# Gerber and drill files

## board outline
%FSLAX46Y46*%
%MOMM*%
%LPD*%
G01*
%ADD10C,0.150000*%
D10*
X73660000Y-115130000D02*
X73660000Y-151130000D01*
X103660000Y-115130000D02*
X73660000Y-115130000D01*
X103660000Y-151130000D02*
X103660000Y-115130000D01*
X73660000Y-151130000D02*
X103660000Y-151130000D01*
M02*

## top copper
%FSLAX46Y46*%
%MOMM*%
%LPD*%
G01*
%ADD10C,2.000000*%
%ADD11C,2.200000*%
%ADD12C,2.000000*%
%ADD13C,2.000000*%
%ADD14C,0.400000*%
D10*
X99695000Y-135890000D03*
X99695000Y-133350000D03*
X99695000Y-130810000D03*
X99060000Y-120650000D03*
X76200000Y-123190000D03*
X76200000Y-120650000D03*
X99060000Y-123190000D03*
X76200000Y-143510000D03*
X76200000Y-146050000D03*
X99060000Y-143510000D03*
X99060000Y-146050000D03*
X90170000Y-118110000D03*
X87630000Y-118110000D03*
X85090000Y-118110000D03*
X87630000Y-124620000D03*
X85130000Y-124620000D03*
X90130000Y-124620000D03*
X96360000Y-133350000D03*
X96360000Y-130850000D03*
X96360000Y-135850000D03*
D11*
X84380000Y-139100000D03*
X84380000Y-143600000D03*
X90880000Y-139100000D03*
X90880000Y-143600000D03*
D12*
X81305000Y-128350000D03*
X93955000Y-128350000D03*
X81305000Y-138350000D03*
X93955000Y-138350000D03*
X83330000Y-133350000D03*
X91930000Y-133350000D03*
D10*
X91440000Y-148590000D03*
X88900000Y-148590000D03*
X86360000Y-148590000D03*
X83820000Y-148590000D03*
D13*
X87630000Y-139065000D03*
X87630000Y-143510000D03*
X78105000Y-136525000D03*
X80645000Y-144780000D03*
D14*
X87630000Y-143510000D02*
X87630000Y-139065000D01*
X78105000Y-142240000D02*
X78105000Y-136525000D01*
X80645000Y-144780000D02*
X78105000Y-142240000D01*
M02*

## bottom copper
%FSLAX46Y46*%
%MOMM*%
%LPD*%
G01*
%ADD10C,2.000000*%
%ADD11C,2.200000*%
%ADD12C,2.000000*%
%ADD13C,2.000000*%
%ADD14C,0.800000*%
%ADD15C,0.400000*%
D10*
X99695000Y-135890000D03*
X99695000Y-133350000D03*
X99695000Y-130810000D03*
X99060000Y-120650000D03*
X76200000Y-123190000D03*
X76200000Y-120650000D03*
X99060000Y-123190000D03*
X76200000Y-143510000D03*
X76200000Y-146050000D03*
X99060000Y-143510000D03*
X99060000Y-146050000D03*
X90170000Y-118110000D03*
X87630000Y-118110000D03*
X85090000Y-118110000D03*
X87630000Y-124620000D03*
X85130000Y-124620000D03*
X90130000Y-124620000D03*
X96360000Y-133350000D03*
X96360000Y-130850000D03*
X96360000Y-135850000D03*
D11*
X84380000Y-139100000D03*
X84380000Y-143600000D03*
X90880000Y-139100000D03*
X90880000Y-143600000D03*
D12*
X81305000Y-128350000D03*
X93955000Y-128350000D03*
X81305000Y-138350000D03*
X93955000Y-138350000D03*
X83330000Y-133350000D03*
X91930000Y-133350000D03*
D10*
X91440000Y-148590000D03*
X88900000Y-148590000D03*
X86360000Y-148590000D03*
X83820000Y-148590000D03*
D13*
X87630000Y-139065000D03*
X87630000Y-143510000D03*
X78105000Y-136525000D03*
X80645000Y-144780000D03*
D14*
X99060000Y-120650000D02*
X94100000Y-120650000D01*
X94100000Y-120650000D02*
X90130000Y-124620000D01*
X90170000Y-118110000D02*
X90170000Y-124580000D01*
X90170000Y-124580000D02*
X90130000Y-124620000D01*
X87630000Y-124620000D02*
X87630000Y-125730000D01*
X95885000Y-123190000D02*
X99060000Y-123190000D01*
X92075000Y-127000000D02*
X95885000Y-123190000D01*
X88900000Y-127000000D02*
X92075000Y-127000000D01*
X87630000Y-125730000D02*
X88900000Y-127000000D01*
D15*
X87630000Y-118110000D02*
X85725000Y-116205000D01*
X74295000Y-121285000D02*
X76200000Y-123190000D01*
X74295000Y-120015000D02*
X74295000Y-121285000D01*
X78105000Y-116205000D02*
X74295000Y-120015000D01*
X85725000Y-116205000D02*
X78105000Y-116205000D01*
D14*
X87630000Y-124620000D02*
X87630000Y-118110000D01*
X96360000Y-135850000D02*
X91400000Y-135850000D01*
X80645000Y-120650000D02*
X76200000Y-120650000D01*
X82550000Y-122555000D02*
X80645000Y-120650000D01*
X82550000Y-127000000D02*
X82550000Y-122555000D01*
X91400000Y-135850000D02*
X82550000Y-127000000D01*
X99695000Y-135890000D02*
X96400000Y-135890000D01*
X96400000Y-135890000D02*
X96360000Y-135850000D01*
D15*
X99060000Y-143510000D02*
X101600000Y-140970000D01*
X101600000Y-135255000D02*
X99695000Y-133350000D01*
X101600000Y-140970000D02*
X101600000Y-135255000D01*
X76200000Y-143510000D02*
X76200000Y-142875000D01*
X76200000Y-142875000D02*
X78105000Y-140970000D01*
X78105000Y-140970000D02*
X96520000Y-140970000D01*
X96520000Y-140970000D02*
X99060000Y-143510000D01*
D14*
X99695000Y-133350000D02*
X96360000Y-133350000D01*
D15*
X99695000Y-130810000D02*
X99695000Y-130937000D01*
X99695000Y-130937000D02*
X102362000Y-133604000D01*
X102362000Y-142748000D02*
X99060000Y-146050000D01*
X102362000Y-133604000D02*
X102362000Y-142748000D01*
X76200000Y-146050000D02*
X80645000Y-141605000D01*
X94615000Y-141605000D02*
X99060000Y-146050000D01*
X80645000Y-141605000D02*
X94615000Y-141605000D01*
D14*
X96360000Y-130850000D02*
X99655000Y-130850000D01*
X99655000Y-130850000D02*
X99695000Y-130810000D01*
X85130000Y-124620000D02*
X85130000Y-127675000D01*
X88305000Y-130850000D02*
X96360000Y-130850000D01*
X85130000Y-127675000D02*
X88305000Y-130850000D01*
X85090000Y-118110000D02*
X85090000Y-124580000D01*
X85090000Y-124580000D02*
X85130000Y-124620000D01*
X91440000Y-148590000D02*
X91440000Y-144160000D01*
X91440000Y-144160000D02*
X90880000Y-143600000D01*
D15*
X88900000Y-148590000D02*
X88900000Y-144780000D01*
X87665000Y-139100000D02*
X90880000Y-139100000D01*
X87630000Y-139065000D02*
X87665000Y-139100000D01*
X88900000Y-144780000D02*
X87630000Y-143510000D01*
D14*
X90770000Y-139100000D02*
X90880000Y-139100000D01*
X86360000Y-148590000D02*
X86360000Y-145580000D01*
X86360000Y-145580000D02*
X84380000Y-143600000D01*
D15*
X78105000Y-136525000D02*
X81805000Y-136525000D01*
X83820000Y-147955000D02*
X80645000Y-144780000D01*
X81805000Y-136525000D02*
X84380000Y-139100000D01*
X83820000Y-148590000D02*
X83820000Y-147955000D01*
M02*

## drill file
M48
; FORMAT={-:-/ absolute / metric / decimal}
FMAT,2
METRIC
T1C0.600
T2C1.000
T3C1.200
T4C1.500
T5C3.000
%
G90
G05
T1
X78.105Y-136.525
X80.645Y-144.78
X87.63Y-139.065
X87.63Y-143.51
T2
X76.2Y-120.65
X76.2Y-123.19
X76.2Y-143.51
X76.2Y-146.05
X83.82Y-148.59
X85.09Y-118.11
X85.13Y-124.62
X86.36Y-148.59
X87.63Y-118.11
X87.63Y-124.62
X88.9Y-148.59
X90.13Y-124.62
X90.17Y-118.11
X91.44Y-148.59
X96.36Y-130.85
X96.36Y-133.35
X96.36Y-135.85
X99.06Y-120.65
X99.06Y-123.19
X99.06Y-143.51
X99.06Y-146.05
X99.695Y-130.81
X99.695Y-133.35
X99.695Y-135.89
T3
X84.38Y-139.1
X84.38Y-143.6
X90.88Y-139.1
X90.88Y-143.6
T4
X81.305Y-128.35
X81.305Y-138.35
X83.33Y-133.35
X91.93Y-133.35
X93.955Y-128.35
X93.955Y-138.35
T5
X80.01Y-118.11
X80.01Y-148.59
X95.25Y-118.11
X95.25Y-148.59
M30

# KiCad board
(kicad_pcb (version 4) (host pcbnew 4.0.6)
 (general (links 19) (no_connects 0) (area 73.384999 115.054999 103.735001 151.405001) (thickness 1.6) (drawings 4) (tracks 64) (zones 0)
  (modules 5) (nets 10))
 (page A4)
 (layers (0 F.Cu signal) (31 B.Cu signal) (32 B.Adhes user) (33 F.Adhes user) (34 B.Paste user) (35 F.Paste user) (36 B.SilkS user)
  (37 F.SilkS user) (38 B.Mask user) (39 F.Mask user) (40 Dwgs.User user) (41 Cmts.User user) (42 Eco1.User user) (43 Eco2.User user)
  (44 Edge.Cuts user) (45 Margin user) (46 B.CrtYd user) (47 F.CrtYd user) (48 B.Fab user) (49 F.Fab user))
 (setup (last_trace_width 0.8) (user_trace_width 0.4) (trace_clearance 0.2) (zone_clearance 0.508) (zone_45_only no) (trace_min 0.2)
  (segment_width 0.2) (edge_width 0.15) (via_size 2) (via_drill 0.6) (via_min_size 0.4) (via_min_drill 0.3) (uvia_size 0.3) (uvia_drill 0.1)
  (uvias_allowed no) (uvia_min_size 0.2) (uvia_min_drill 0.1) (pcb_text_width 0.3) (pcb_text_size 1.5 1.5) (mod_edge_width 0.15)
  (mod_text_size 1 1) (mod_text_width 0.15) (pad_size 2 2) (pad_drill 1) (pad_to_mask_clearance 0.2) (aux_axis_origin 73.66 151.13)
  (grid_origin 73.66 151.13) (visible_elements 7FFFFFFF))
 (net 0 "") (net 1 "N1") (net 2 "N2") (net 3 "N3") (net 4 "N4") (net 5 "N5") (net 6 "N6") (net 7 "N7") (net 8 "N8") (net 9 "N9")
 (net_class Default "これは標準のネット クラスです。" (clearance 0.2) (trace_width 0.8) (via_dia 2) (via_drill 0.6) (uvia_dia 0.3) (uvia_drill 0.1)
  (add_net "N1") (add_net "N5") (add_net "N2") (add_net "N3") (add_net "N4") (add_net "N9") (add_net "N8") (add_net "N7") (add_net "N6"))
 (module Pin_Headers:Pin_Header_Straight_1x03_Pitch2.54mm (layer F.Cu) (at 99.695 135.89 180)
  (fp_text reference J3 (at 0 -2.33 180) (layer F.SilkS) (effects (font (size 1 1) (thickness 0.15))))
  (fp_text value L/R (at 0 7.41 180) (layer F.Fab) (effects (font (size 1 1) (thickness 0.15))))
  (pad 1 thru_hole circle (at 0 0 180) (size 2 2) (drill 1) (layers *.Cu *.Mask) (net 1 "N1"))
  (pad 2 thru_hole circle (at 0 2.54 180) (size 2 2) (drill 1) (layers *.Cu *.Mask) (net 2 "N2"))
  (pad 3 thru_hole circle (at 0 5.08 180) (size 2 2) (drill 1) (layers *.Cu *.Mask) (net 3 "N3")))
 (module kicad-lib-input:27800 (layer F.Cu) (at 87.63 133.35)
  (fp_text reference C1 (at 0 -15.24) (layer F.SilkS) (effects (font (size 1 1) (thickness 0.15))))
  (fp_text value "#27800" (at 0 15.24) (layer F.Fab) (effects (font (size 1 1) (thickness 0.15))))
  (pad 5 thru_hole circle (at 11.43 -12.7) (size 2 2) (drill 1) (layers *.Cu *.Mask) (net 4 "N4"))
  (pad 2 thru_hole circle (at -11.43 -10.16) (size 2 2) (drill 1) (layers *.Cu *.Mask) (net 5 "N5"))
  (pad 1 thru_hole circle (at -11.43 -12.7) (size 2 2) (drill 1) (layers *.Cu *.Mask) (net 1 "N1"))
  (pad 6 thru_hole circle (at 11.43 -10.16) (size 2 2) (drill 1) (layers *.Cu *.Mask) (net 5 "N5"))
  (pad 3 thru_hole circle (at -11.43 10.16) (size 2 2) (drill 1) (layers *.Cu *.Mask) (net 2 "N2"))
  (pad 4 thru_hole circle (at -11.43 12.7) (size 2 2) (drill 1) (layers *.Cu *.Mask) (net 3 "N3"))
  (pad 7 thru_hole circle (at 11.43 10.16) (size 2 2) (drill 1) (layers *.Cu *.Mask) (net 2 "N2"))
  (pad 8 thru_hole circle (at 11.43 12.7) (size 2 2) (drill 1) (layers *.Cu *.Mask) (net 3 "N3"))
  (pad "" np_thru_hole circle (at 7.62 -15.24) (size 3 3) (drill 3) (layers *.Cu *.Mask))
  (pad "" np_thru_hole circle (at -7.62 -15.24) (size 3 3) (drill 3) (layers *.Cu *.Mask))
  (pad "" np_thru_hole circle (at -7.62 15.24) (size 3 3) (drill 3) (layers *.Cu *.Mask))
  (pad "" np_thru_hole circle (at 7.62 15.24) (size 3 3) (drill 3) (layers *.Cu *.Mask)))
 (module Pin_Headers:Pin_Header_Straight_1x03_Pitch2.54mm (layer F.Cu) (at 90.17 118.11 270)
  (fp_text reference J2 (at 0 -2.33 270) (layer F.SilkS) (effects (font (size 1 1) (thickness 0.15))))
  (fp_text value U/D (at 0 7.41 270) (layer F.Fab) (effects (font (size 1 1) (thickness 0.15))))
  (pad 1 thru_hole circle (at 0 0 270) (size 2 2) (drill 1) (layers *.Cu *.Mask) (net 4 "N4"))
  (pad 2 thru_hole circle (at 0 2.54 270) (size 2 2) (drill 1) (layers *.Cu *.Mask) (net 5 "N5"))
  (pad 3 thru_hole circle (at 0 5.08 270) (size 2 2) (drill 1) (layers *.Cu *.Mask) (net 3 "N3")))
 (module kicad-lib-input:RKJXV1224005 (layer F.Cu) (at 87.63 133.35)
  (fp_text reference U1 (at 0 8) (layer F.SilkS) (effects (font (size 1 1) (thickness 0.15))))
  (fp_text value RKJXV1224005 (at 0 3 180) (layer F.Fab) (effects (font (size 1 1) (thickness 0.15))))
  (pad 5 thru_hole circle (at 0 -8.73) (size 2 2) (drill 1) (layers *.Cu *.Mask) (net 5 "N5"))
  (pad 6 thru_hole circle (at -2.5 -8.73) (size 2 2) (drill 1) (layers *.Cu *.Mask) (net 3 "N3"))
  (pad 4 thru_hole circle (at 2.5 -8.73) (size 2 2) (drill 1) (layers *.Cu *.Mask) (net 4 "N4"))
  (pad 2 thru_hole circle (at 8.73 0) (size 2 2) (drill 1) (layers *.Cu *.Mask) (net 2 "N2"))
  (pad 3 thru_hole circle (at 8.73 -2.5) (size 2 2) (drill 1) (layers *.Cu *.Mask) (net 3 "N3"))
  (pad 1 thru_hole circle (at 8.73 2.5) (size 2 2) (drill 1) (layers *.Cu *.Mask) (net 1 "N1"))
  (pad 7 thru_hole circle (at -3.25 5.75) (size 2.2 2.2) (drill 1.2) (layers *.Cu *.Mask) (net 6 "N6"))
  (pad 8 thru_hole circle (at -3.25 10.25) (size 2.2 2.2) (drill 1.2) (layers *.Cu *.Mask) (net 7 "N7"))
  (pad 9 thru_hole circle (at 3.25 5.75) (size 2.2 2.2) (drill 1.2) (layers *.Cu *.Mask) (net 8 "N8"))
  (pad 10 thru_hole circle (at 3.25 10.25) (size 2.2 2.2) (drill 1.2) (layers *.Cu *.Mask) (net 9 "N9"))
  (pad "" np_thru_hole circle (at -6.325 -5) (size 2 2) (drill 1.5) (layers *.Cu *.Mask))
  (pad "" np_thru_hole circle (at 6.325 -5) (size 2 2) (drill 1.5) (layers *.Cu *.Mask))
  (pad "" np_thru_hole circle (at -6.325 5) (size 2 2) (drill 1.5) (layers *.Cu *.Mask))
  (pad "" np_thru_hole circle (at 6.325 5) (size 2 2) (drill 1.5) (layers *.Cu *.Mask))
  (pad "" np_thru_hole circle (at -4.3 0) (size 2 2) (drill 1.5) (layers *.Cu *.Mask))
  (pad "" np_thru_hole circle (at 4.3 0) (size 2 2) (drill 1.5) (layers *.Cu *.Mask)))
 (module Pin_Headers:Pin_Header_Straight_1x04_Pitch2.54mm (layer F.Cu) (at 91.44 148.59 270)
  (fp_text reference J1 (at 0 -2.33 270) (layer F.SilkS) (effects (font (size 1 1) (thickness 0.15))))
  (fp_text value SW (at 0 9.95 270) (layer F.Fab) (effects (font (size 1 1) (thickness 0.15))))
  (pad 1 thru_hole circle (at 0 0 270) (size 2 2) (drill 1) (layers *.Cu *.Mask) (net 9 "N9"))
  (pad 2 thru_hole circle (at 0 2.54 270) (size 2 2) (drill 1) (layers *.Cu *.Mask) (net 8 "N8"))
  (pad 3 thru_hole circle (at 0 5.08 270) (size 2 2) (drill 1) (layers *.Cu *.Mask) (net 7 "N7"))
  (pad 4 thru_hole circle (at 0 7.62 270) (size 2 2) (drill 1) (layers *.Cu *.Mask) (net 6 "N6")))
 (gr_line (start 73.66 115.13) (end 73.66 151.13) (angle 90) (layer Edge.Cuts) (width 0.15))
 (gr_line (start 103.66 115.13) (end 73.66 115.13) (angle 90) (layer Edge.Cuts) (width 0.15))
 (gr_line (start 103.66 151.13) (end 103.66 115.13) (angle 90) (layer Edge.Cuts) (width 0.15))
 (gr_line (start 73.66 151.13) (end 103.66 151.13) (angle 90) (layer Edge.Cuts) (width 0.15))
 (segment (start 99.06 120.65) (end 94.1 120.65) (width 0.8) (layer B.Cu) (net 4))
 (segment (start 94.1 120.65) (end 90.13 124.62) (width 0.8) (layer B.Cu) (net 4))
 (segment (start 90.17 118.11) (end 90.17 124.58) (width 0.8) (layer B.Cu) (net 4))
 (segment (start 90.17 124.58) (end 90.13 124.62) (width 0.8) (layer B.Cu) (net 4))
 (segment (start 87.63 124.62) (end 87.63 125.73) (width 0.8) (layer B.Cu) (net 5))
 (segment (start 95.885 123.19) (end 99.06 123.19) (width 0.8) (layer B.Cu) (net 5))
 (segment (start 92.075 127) (end 95.885 123.19) (width 0.8) (layer B.Cu) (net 5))
 (segment (start 88.9 127) (end 92.075 127) (width 0.8) (layer B.Cu) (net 5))
 (segment (start 87.63 125.73) (end 88.9 127) (width 0.8) (layer B.Cu) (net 5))
 (segment (start 87.63 118.11) (end 85.725 116.205) (width 0.4) (layer B.Cu) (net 5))
 (segment (start 74.295 121.285) (end 76.2 123.19) (width 0.4) (layer B.Cu) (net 5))
 (segment (start 74.295 120.015) (end 74.295 121.285) (width 0.4) (layer B.Cu) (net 5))
 (segment (start 78.105 116.205) (end 74.295 120.015) (width 0.4) (layer B.Cu) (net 5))
 (segment (start 85.725 116.205) (end 78.105 116.205) (width 0.4) (layer B.Cu) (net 5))
 (segment (start 87.63 124.62) (end 87.63 118.11) (width 0.8) (layer B.Cu) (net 5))
 (segment (start 96.36 135.85) (end 91.4 135.85) (width 0.8) (layer B.Cu) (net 1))
 (segment (start 80.645 120.65) (end 76.2 120.65) (width 0.8) (layer B.Cu) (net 1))
 (segment (start 82.55 122.555) (end 80.645 120.65) (width 0.8) (layer B.Cu) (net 1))
 (segment (start 82.55 127) (end 82.55 122.555) (width 0.8) (layer B.Cu) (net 1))
 (segment (start 91.4 135.85) (end 82.55 127) (width 0.8) (layer B.Cu) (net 1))
 (segment (start 99.695 135.89) (end 96.4 135.89) (width 0.8) (layer B.Cu) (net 1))
 (segment (start 96.4 135.89) (end 96.36 135.85) (width 0.8) (layer B.Cu) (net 1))
 (segment (start 99.06 143.51) (end 101.6 140.97) (width 0.4) (layer B.Cu) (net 2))
 (segment (start 101.6 135.255) (end 99.695 133.35) (width 0.4) (layer B.Cu) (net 2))
 (segment (start 101.6 140.97) (end 101.6 135.255) (width 0.4) (layer B.Cu) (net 2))
 (segment (start 76.2 143.51) (end 76.2 142.875) (width 0.4) (layer B.Cu) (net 2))
 (segment (start 76.2 142.875) (end 78.105 140.97) (width 0.4) (layer B.Cu) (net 2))
 (segment (start 78.105 140.97) (end 96.52 140.97) (width 0.4) (layer B.Cu) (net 2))
 (segment (start 96.52 140.97) (end 99.06 143.51) (width 0.4) (layer B.Cu) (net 2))
 (segment (start 99.695 133.35) (end 96.36 133.35) (width 0.8) (layer B.Cu) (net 2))
 (segment (start 99.695 130.81) (end 99.695 130.937) (width 0.4) (layer B.Cu) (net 3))
 (segment (start 99.695 130.937) (end 102.362 133.604) (width 0.4) (layer B.Cu) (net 3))
 (segment (start 102.362 142.748) (end 99.06 146.05) (width 0.4) (layer B.Cu) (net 3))
 (segment (start 102.362 133.604) (end 102.362 142.748) (width 0.4) (layer B.Cu) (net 3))
 (segment (start 76.2 146.05) (end 80.645 141.605) (width 0.4) (layer B.Cu) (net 3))
 (segment (start 94.615 141.605) (end 99.06 146.05) (width 0.4) (layer B.Cu) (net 3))
 (segment (start 80.645 141.605) (end 94.615 141.605) (width 0.4) (layer B.Cu) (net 3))
 (segment (start 96.36 130.85) (end 99.655 130.85) (width 0.8) (layer B.Cu) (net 3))
 (segment (start 99.655 130.85) (end 99.695 130.81) (width 0.8) (layer B.Cu) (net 3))
 (segment (start 85.13 124.62) (end 85.13 127.675) (width 0.8) (layer B.Cu) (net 3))
 (segment (start 88.305 130.85) (end 96.36 130.85) (width 0.8) (layer B.Cu) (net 3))
 (segment (start 85.13 127.675) (end 88.305 130.85) (width 0.8) (layer B.Cu) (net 3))
 (segment (start 85.09 118.11) (end 85.09 124.58) (width 0.8) (layer B.Cu) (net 3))
 (segment (start 85.09 124.58) (end 85.13 124.62) (width 0.8) (layer B.Cu) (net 3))
 (segment (start 91.44 148.59) (end 91.44 144.16) (width 0.8) (layer B.Cu) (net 9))
 (segment (start 91.44 144.16) (end 90.88 143.6) (width 0.8) (layer B.Cu) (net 9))
 (segment (start 88.9 148.59) (end 88.9 144.78) (width 0.4) (layer B.Cu) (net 8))
 (segment (start 87.665 139.1) (end 90.88 139.1) (width 0.4) (layer B.Cu) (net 8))
 (segment (start 87.63 139.065) (end 87.665 139.1) (width 0.4) (layer B.Cu) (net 8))
 (via (at 87.63 139.065) (size 2) (drill 0.6) (layers F.Cu B.Cu) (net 8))
 (segment (start 87.63 143.51) (end 87.63 139.065) (width 0.4) (layer F.Cu) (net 8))
 (via (at 87.63 143.51) (size 2) (drill 0.6) (layers F.Cu B.Cu) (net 8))
 (segment (start 88.9 144.78) (end 87.63 143.51) (width 0.4) (layer B.Cu) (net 8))
 (segment (start 90.77 139.1) (end 90.88 139.1) (width 0.8) (layer B.Cu) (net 8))
 (segment (start 86.36 148.59) (end 86.36 145.58) (width 0.8) (layer B.Cu) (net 7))
 (segment (start 86.36 145.58) (end 84.38 143.6) (width 0.8) (layer B.Cu) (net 7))
 (segment (start 78.105 136.525) (end 81.805 136.525) (width 0.4) (layer B.Cu) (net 6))
 (via (at 78.105 136.525) (size 2) (drill 0.6) (layers F.Cu B.Cu) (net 6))
 (segment (start 78.105 142.24) (end 78.105 136.525) (width 0.4) (layer F.Cu) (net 6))
 (segment (start 80.645 144.78) (end 78.105 142.24) (width 0.4) (layer F.Cu) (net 6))
 (via (at 80.645 144.78) (size 2) (drill 0.6) (layers F.Cu B.Cu) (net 6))
 (segment (start 83.82 147.955) (end 80.645 144.78) (width 0.4) (layer B.Cu) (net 6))
 (segment (start 81.805 136.525) (end 84.38 139.1) (width 0.4) (layer B.Cu) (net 6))
 (segment (start 83.82 148.59) (end 83.82 147.955) (width 0.4) (layer B.Cu) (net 6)))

